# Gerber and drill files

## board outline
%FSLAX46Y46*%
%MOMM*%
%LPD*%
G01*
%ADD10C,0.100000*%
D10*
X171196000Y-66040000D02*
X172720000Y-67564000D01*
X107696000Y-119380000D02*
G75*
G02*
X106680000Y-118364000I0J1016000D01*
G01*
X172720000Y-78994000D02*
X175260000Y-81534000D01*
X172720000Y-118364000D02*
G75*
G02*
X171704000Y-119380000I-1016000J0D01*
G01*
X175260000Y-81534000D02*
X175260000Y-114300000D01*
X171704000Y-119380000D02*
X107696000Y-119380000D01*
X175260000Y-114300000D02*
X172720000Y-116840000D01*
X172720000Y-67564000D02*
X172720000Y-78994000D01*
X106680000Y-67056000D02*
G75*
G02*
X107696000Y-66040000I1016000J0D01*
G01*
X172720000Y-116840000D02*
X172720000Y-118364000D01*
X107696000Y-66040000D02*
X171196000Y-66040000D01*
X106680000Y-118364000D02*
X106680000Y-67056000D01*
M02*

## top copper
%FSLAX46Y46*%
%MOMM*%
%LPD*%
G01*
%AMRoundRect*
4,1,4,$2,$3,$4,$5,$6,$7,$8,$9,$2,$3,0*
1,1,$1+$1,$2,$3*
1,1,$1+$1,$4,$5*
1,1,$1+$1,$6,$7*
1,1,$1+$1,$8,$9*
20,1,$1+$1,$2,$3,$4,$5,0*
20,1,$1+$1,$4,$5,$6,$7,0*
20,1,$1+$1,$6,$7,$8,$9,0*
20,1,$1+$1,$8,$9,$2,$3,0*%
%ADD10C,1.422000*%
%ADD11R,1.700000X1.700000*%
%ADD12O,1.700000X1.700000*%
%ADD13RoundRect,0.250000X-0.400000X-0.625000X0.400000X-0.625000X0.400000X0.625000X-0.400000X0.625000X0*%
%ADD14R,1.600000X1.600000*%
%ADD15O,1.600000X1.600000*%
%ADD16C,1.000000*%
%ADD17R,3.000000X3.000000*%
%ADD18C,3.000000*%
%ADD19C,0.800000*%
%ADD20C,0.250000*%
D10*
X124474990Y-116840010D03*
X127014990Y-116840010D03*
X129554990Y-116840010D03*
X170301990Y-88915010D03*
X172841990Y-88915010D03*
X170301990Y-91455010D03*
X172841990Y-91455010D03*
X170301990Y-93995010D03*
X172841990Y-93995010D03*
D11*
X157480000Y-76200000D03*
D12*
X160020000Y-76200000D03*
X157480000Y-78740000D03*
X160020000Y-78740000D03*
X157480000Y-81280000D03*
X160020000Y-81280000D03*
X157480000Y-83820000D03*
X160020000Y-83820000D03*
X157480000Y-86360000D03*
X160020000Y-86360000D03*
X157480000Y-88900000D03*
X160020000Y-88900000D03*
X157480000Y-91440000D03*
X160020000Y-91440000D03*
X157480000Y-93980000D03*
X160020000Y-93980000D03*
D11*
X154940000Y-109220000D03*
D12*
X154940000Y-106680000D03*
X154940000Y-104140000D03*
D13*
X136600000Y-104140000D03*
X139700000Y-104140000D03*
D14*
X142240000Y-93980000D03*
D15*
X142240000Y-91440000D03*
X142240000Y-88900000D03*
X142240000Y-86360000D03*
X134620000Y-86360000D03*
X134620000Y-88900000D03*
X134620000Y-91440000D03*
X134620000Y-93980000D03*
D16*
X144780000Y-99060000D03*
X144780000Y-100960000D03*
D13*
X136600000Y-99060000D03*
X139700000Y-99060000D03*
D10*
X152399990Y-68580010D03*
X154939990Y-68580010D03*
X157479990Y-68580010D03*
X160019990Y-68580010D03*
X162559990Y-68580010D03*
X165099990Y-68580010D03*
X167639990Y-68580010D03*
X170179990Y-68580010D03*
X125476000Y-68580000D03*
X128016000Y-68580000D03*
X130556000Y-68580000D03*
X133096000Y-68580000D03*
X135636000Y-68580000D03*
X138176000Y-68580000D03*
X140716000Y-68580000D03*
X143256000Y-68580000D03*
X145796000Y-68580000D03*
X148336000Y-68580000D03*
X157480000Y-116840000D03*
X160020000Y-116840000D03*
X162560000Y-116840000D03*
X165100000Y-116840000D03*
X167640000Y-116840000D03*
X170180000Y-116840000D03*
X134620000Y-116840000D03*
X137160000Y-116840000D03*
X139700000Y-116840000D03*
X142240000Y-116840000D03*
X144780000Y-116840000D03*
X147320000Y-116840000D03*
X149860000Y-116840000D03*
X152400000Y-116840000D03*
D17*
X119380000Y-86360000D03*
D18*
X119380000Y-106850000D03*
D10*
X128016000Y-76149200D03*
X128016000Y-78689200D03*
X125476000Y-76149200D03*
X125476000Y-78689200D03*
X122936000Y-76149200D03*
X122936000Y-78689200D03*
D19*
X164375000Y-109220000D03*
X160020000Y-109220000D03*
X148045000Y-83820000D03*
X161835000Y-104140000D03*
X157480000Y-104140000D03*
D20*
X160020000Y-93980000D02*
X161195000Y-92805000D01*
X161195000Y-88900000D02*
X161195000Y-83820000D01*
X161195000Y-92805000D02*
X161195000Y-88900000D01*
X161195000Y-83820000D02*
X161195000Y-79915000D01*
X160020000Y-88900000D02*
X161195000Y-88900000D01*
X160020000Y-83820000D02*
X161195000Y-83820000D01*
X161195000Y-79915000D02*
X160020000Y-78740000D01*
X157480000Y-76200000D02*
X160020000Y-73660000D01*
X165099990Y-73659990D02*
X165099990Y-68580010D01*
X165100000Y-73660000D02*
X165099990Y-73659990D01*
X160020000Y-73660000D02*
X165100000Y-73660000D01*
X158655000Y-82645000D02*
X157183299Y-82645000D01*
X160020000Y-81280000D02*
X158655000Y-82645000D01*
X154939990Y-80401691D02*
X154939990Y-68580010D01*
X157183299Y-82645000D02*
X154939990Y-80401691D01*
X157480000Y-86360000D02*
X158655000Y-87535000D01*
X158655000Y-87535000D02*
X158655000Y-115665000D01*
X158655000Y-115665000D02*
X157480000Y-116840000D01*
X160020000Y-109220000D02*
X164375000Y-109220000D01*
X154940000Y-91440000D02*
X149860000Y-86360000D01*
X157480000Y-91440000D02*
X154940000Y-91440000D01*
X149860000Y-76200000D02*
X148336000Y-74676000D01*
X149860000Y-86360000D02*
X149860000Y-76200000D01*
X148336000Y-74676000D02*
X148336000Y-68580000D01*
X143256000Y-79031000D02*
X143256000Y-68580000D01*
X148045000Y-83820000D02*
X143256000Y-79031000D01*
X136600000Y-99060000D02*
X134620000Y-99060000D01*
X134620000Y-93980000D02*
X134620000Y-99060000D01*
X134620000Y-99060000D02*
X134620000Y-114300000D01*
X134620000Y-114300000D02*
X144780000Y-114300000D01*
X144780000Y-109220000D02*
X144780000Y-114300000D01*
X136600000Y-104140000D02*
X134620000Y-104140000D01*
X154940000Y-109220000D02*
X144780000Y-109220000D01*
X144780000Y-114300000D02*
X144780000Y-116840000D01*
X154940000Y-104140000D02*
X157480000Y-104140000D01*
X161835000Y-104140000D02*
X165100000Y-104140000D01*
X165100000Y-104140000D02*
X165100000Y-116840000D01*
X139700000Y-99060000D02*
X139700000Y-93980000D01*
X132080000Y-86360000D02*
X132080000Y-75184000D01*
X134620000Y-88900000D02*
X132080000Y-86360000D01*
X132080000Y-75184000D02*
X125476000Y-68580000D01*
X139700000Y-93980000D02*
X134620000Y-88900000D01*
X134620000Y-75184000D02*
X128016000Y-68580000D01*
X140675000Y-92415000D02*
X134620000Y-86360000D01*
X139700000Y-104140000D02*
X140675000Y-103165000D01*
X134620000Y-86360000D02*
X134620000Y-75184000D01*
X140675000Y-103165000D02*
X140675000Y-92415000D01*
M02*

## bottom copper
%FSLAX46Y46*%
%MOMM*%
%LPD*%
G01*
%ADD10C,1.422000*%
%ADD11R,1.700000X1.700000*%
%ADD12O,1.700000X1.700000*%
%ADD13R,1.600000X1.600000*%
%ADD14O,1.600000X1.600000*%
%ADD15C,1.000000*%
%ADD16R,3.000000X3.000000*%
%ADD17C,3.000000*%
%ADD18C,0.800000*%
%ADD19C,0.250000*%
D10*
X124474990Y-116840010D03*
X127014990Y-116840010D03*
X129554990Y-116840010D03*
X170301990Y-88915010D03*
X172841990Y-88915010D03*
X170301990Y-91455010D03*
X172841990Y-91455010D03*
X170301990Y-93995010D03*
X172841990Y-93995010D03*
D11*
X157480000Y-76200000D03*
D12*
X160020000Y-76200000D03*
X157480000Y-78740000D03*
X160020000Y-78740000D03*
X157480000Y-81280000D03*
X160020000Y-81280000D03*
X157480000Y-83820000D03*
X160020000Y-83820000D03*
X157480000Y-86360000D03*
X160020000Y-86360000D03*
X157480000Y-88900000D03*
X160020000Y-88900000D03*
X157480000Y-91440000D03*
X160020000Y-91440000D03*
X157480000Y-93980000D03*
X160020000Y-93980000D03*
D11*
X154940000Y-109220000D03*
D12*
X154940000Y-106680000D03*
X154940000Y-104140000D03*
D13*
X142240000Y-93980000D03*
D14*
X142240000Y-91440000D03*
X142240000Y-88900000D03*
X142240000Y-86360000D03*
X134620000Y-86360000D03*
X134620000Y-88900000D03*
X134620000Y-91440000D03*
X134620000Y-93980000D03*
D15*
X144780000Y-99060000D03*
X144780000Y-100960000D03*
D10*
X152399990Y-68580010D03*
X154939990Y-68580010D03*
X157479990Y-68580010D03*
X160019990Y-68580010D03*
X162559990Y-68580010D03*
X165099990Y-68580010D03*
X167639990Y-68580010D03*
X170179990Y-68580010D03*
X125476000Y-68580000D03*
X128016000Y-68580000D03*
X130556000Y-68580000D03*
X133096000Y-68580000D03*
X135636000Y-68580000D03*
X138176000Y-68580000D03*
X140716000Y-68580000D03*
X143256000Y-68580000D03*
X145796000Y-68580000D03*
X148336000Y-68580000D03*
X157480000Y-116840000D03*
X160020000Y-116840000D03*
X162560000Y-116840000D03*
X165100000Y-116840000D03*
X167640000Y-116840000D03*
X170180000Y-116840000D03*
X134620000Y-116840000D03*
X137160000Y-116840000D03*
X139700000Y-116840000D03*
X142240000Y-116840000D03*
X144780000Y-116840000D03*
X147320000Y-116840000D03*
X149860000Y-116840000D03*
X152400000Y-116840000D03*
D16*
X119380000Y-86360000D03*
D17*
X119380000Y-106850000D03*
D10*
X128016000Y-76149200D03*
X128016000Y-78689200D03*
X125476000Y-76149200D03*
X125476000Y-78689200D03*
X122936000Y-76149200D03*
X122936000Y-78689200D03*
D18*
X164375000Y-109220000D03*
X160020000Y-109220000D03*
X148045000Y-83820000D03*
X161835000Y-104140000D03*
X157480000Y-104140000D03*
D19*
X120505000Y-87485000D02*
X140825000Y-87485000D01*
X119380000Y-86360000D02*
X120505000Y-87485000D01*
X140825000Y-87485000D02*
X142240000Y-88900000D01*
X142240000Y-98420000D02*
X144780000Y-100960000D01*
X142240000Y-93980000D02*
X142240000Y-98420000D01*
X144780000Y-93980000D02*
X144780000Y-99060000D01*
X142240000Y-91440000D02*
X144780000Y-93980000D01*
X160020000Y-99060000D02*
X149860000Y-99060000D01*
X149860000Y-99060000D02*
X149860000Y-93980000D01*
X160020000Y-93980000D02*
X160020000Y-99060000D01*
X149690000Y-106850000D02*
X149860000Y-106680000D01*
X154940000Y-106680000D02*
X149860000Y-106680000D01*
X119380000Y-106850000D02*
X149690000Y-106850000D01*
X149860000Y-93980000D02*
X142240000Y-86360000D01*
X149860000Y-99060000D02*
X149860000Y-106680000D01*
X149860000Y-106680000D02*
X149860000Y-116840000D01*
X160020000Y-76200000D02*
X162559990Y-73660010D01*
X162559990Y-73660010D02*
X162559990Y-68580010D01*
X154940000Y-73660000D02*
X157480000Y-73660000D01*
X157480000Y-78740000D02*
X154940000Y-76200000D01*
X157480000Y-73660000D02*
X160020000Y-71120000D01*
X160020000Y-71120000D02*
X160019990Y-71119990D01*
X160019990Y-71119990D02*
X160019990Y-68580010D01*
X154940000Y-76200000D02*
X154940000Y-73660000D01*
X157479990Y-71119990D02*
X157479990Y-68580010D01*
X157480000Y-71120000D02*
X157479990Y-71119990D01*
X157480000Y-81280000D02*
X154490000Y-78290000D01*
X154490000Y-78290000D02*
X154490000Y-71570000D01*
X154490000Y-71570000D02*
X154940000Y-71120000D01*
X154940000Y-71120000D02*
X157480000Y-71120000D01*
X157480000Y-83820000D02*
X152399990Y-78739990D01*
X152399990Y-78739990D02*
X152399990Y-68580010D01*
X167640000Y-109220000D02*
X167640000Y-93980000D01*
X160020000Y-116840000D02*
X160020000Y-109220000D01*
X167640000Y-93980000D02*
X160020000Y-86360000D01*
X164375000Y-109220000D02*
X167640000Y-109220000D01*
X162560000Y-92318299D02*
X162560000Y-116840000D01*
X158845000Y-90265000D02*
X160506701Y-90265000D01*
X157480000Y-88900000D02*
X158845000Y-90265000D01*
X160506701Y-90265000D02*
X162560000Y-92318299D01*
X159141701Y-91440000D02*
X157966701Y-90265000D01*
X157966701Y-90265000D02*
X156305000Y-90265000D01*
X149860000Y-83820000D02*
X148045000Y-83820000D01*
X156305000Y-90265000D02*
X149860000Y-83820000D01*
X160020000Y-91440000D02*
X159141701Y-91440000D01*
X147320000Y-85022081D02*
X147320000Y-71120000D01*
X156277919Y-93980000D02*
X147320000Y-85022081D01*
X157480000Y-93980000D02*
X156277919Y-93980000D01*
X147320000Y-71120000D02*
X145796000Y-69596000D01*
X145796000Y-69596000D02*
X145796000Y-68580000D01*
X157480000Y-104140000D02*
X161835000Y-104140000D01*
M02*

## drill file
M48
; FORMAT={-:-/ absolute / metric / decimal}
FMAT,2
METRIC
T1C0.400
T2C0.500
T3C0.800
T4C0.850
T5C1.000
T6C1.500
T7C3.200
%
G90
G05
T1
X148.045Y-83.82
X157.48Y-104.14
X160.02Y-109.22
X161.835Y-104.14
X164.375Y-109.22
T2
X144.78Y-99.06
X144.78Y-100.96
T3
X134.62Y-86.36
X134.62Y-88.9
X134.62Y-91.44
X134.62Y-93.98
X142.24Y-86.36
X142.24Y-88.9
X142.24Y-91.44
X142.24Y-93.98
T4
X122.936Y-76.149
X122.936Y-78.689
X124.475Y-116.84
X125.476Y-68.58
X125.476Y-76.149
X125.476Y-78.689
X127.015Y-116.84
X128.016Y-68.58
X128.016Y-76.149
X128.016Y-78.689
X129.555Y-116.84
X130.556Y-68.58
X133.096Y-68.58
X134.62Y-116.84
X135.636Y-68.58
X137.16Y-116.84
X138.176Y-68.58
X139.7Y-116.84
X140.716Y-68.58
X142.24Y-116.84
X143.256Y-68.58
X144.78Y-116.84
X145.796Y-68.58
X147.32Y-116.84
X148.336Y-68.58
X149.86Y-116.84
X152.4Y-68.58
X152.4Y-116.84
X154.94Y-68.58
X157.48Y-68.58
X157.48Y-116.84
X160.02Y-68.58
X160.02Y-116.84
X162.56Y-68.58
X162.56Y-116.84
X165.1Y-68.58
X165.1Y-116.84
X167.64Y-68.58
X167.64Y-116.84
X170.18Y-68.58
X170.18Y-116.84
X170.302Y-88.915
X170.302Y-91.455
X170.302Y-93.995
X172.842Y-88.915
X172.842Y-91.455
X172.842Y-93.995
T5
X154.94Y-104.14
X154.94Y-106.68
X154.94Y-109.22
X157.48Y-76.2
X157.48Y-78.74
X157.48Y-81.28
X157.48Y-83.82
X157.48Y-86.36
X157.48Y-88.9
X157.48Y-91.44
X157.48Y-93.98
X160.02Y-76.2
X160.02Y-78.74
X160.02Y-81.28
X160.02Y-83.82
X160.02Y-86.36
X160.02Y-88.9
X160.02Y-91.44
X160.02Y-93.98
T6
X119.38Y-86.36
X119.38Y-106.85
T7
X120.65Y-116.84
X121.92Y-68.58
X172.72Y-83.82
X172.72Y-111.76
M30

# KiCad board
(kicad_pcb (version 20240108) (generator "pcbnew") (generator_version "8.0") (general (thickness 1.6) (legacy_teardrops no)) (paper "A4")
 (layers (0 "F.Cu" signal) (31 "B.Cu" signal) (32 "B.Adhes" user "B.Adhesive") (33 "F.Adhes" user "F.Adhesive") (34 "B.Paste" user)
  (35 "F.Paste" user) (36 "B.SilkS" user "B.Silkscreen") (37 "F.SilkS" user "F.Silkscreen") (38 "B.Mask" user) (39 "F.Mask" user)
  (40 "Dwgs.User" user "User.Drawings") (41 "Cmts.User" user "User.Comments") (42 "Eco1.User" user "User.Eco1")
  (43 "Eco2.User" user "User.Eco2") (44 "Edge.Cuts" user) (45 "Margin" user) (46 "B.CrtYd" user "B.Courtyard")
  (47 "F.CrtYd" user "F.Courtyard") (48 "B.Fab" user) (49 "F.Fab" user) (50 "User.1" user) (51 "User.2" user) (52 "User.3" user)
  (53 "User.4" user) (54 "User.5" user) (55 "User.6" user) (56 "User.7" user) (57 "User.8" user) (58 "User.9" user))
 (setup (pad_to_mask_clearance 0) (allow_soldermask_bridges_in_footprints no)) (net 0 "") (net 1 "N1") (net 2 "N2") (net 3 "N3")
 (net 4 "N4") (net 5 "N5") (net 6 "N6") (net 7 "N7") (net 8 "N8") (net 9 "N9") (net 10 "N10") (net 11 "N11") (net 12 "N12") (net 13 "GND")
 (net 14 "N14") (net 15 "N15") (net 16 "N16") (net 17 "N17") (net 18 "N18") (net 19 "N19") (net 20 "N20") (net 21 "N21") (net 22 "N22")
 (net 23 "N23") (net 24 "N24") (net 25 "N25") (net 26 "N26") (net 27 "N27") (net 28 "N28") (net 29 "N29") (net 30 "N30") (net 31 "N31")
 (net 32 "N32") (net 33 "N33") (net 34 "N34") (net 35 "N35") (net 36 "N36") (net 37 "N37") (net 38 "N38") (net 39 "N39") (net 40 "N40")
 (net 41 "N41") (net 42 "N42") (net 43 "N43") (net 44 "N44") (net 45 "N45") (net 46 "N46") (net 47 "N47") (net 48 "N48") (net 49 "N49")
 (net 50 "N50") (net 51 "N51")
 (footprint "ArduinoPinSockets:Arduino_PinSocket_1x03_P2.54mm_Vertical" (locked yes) (layer "F.Cu") (at 124.47499 116.84001 90)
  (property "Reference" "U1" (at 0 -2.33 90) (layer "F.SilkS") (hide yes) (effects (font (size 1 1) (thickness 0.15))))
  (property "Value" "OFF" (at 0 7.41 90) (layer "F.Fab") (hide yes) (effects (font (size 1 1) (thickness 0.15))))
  (pad "1" thru_hole circle (at 0 0 90) (size 1.422 1.422) (drill 0.85) (layers "*.Cu" "*.Mask") (remove_unused_layers no) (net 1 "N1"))
  (pad "2" thru_hole circle (at 0 2.54 90) (size 1.422 1.422) (drill 0.85) (layers "*.Cu" "*.Mask") (remove_unused_layers no) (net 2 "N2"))
  (pad "3" thru_hole circle (at 0 5.08 90) (size 1.422 1.422) (drill 0.85) (layers "*.Cu" "*.Mask") (remove_unused_layers no) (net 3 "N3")))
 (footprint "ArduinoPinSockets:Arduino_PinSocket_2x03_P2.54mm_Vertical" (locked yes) (layer "F.Cu") (at 170.30199 88.91501)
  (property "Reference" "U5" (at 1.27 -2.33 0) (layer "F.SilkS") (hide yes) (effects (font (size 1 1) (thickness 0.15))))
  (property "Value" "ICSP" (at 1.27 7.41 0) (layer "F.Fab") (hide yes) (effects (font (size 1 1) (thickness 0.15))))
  (pad "1" thru_hole circle (at 0 0) (size 1.422 1.422) (drill 0.85) (layers "*.Cu" "*.Mask") (remove_unused_layers no) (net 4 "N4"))
  (pad "2" thru_hole circle (at 2.54 0) (size 1.422 1.422) (drill 0.85) (layers "*.Cu" "*.Mask") (remove_unused_layers no) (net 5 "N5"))
  (pad "3" thru_hole circle (at 0 2.54) (size 1.422 1.422) (drill 0.85) (layers "*.Cu" "*.Mask") (remove_unused_layers no) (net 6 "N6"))
  (pad "4" thru_hole circle (at 2.54 2.54) (size 1.422 1.422) (drill 0.85) (layers "*.Cu" "*.Mask") (remove_unused_layers no) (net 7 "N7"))
  (pad "5" thru_hole circle (at 0 5.08) (size 1.422 1.422) (drill 0.85) (layers "*.Cu" "*.Mask") (remove_unused_layers no) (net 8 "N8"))
  (pad "6" thru_hole circle (at 2.54 5.08) (size 1.422 1.422) (drill 0.85) (layers "*.Cu" "*.Mask") (remove_unused_layers no) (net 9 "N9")))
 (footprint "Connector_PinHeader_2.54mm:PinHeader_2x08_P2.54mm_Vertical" (layer "F.Cu") (at 157.48 76.2)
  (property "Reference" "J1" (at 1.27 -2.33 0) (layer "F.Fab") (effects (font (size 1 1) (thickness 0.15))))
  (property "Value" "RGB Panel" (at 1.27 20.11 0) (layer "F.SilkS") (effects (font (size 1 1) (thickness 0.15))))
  (pad "1" thru_hole rect (at 0 0) (size 1.7 1.7) (drill 1) (layers "*.Cu" "*.Mask") (remove_unused_layers no) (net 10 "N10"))
  (pad "2" thru_hole oval (at 2.54 0) (size 1.7 1.7) (drill 1) (layers "*.Cu" "*.Mask") (remove_unused_layers no) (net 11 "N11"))
  (pad "3" thru_hole oval (at 0 2.54) (size 1.7 1.7) (drill 1) (layers "*.Cu" "*.Mask") (remove_unused_layers no) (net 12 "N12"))
  (pad "4" thru_hole oval (at 2.54 2.54) (size 1.7 1.7) (drill 1) (layers "*.Cu" "*.Mask") (remove_unused_layers no) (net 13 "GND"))
  (pad "5" thru_hole oval (at 0 5.08) (size 1.7 1.7) (drill 1) (layers "*.Cu" "*.Mask") (remove_unused_layers no) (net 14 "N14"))
  (pad "6" thru_hole oval (at 2.54 5.08) (size 1.7 1.7) (drill 1) (layers "*.Cu" "*.Mask") (remove_unused_layers no) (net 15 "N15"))
  (pad "7" thru_hole oval (at 0 7.62) (size 1.7 1.7) (drill 1) (layers "*.Cu" "*.Mask") (remove_unused_layers no) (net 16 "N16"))
  (pad "8" thru_hole oval (at 2.54 7.62) (size 1.7 1.7) (drill 1) (layers "*.Cu" "*.Mask") (remove_unused_layers no) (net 13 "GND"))
  (pad "9" thru_hole oval (at 0 10.16) (size 1.7 1.7) (drill 1) (layers "*.Cu" "*.Mask") (remove_unused_layers no) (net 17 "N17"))
  (pad "10" thru_hole oval (at 2.54 10.16) (size 1.7 1.7) (drill 1) (layers "*.Cu" "*.Mask") (remove_unused_layers no) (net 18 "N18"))
  (pad "11" thru_hole oval (at 0 12.7) (size 1.7 1.7) (drill 1) (layers "*.Cu" "*.Mask") (remove_unused_layers no) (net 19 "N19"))
  (pad "12" thru_hole oval (at 2.54 12.7) (size 1.7 1.7) (drill 1) (layers "*.Cu" "*.Mask") (remove_unused_layers no) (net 15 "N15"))
  (pad "13" thru_hole oval (at 0 15.24) (size 1.7 1.7) (drill 1) (layers "*.Cu" "*.Mask") (remove_unused_layers no) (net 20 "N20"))
  (pad "14" thru_hole oval (at 2.54 15.24) (size 1.7 1.7) (drill 1) (layers "*.Cu" "*.Mask") (remove_unused_layers no) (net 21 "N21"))
  (pad "15" thru_hole oval (at 0 17.78) (size 1.7 1.7) (drill 1) (layers "*.Cu" "*.Mask") (remove_unused_layers no) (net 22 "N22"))
  (pad "16" thru_hole oval (at 2.54 17.78) (size 1.7 1.7) (drill 1) (layers "*.Cu" "*.Mask") (remove_unused_layers no) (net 13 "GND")))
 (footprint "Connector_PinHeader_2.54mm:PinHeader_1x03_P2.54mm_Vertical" (layer "F.Cu") (at 154.94 109.22 180)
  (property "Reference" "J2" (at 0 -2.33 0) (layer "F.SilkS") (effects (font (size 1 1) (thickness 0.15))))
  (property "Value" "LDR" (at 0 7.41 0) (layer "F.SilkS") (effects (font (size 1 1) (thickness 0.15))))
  (pad "1" thru_hole rect (at 0 0 180) (size 1.7 1.7) (drill 1) (layers "*.Cu" "*.Mask") (remove_unused_layers no) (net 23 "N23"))
  (pad "2" thru_hole oval (at 0 2.54 180) (size 1.7 1.7) (drill 1) (layers "*.Cu" "*.Mask") (remove_unused_layers no) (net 13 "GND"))
  (pad "3" thru_hole oval (at 0 5.08 180) (size 1.7 1.7) (drill 1) (layers "*.Cu" "*.Mask") (remove_unused_layers no) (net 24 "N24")))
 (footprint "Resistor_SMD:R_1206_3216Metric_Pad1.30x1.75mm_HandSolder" (layer "F.Cu") (at 138.15 104.14)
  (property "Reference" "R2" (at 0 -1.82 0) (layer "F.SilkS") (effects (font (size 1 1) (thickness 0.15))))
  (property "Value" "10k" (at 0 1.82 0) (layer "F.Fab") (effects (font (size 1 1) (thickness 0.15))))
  (pad "1" smd roundrect (at -1.55 0) (size 1.3 1.75) (layers "F.Cu" "F.Paste" "F.Mask") (roundrect_rratio 0.1923076923) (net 23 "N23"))
  (pad "2" smd roundrect (at 1.55 0) (size 1.3 1.75) (layers "F.Cu" "F.Paste" "F.Mask") (roundrect_rratio 0.1923076923) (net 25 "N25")))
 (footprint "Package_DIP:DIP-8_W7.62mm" (layer "F.Cu") (at 142.24 93.98 180)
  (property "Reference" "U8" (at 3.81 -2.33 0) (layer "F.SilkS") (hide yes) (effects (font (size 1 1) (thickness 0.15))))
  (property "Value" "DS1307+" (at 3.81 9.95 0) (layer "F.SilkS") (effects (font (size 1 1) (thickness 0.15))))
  (pad "1" thru_hole rect (at 0 0 180) (size 1.6 1.6) (drill 0.8) (layers "*.Cu" "*.Mask") (remove_unused_layers no) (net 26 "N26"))
  (pad "2" thru_hole oval (at 0 2.54 180) (size 1.6 1.6) (drill 0.8) (layers "*.Cu" "*.Mask") (remove_unused_layers no) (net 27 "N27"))
  (pad "3" thru_hole oval (at 0 5.08 180) (size 1.6 1.6) (drill 0.8) (layers "*.Cu" "*.Mask") (remove_unused_layers no) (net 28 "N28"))
  (pad "4" thru_hole oval (at 0 7.62 180) (size 1.6 1.6) (drill 0.8) (layers "*.Cu" "*.Mask") (remove_unused_layers no) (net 13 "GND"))
  (pad "5" thru_hole oval (at 7.62 7.62 180) (size 1.6 1.6) (drill 0.8) (layers "*.Cu" "*.Mask") (remove_unused_layers no) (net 25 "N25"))
  (pad "6" thru_hole oval (at 7.62 5.08 180) (size 1.6 1.6) (drill 0.8) (layers "*.Cu" "*.Mask") (remove_unused_layers no) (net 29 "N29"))
  (pad "7" thru_hole oval (at 7.62 2.54 180) (size 1.6 1.6) (drill 0.8) (layers "*.Cu" "*.Mask") (remove_unused_layers no) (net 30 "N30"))
  (pad "8" thru_hole oval (at 7.62 0 180) (size 1.6 1.6) (drill 0.8) (layers "*.Cu" "*.Mask") (remove_unused_layers no) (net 23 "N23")))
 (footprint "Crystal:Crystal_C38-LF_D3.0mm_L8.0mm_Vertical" (layer "F.Cu") (at 144.78 99.06 -90)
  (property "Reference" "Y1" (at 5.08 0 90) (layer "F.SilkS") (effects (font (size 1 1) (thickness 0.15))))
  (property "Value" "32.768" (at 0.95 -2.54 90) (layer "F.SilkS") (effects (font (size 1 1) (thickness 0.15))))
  (pad "1" thru_hole circle (at 0 0 270) (size 1 1) (drill 0.5) (layers "*.Cu" "*.Mask") (remove_unused_layers no) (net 27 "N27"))
  (pad "2" thru_hole circle (at 1.9 0 270) (size 1 1) (drill 0.5) (layers "*.Cu" "*.Mask") (remove_unused_layers no) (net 26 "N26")))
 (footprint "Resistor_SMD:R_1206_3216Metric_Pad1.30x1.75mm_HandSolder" (layer "F.Cu") (at 138.15 99.06)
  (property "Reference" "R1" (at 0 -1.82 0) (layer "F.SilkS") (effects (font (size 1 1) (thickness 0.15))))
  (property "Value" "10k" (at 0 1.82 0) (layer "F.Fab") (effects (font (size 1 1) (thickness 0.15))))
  (pad "1" smd roundrect (at -1.55 0) (size 1.3 1.75) (layers "F.Cu" "F.Paste" "F.Mask") (roundrect_rratio 0.1923076923) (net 23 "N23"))
  (pad "2" smd roundrect (at 1.55 0) (size 1.3 1.75) (layers "F.Cu" "F.Paste" "F.Mask") (roundrect_rratio 0.1923076923) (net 29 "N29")))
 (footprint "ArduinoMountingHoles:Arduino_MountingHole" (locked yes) (layer "F.Cu") (at 172.72 83.82001)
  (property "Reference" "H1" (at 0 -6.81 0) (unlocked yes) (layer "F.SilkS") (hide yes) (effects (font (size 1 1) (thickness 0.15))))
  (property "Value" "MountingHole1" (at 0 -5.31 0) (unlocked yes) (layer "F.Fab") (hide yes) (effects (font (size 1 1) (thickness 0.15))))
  (pad "" np_thru_hole circle (at 0 0) (size 3.19989 3.19989) (drill 3.19989) (layers "F&B.Cu" "*.Mask") (solder_mask_margin 0.5)))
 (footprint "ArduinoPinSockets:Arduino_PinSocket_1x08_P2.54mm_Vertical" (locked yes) (layer "F.Cu") (at 152.39999 68.58001 90)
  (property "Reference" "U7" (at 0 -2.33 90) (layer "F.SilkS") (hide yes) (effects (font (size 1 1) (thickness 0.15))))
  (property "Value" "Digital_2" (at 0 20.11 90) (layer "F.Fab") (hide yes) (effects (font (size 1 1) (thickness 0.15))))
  (pad "11" thru_hole circle (at 0 0 90) (size 1.422 1.422) (drill 0.85) (layers "*.Cu" "*.Mask") (remove_unused_layers no) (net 16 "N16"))
  (pad "12" thru_hole circle (at 0 2.54 90) (size 1.422 1.422) (drill 0.85) (layers "*.Cu" "*.Mask") (remove_unused_layers no)
   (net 15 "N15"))
  (pad "13" thru_hole circle (at 0 5.08 90) (size 1.422 1.422) (drill 0.85) (layers "*.Cu" "*.Mask") (remove_unused_layers no)
   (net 14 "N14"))
  (pad "14" thru_hole circle (at 0 7.62 90) (size 1.422 1.422) (drill 0.85) (layers "*.Cu" "*.Mask") (remove_unused_layers no)
   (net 12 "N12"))
  (pad "15" thru_hole circle (at 0 10.16 90) (size 1.422 1.422) (drill 0.85) (layers "*.Cu" "*.Mask") (remove_unused_layers no)
   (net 11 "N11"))
  (pad "16" thru_hole circle (at 0 12.7 90) (size 1.422 1.422) (drill 0.85) (layers "*.Cu" "*.Mask") (remove_unused_layers no)
   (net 10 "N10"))
  (pad "17" thru_hole circle (at 0 15.24 90) (size 1.422 1.422) (drill 0.85) (layers "*.Cu" "*.Mask") (remove_unused_layers no)
   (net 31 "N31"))
  (pad "18" thru_hole circle (at 0 17.78 90) (size 1.422 1.422) (drill 0.85) (layers "*.Cu" "*.Mask") (remove_unused_layers no)
   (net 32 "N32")))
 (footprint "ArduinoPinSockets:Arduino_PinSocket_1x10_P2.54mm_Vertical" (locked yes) (layer "F.Cu") (at 125.476 68.58 90)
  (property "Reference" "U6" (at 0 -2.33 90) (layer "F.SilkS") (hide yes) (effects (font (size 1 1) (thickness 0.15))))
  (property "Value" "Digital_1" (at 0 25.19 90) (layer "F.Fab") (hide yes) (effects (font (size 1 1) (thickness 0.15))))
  (pad "1" thru_hole circle (at 0 0 90) (size 1.422 1.422) (drill 0.85) (layers "*.Cu" "*.Mask") (remove_unused_layers no) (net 29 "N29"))
  (pad "2" thru_hole circle (at 0 2.54 90) (size 1.422 1.422) (drill 0.85) (layers "*.Cu" "*.Mask") (remove_unused_layers no) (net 25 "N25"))
  (pad "3" thru_hole circle (at 0 5.08 90) (size 1.422 1.422) (drill 0.85) (layers "*.Cu" "*.Mask") (remove_unused_layers no) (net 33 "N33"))
  (pad "4" thru_hole circle (at 0 7.62 90) (size 1.422 1.422) (drill 0.85) (layers "*.Cu" "*.Mask") (remove_unused_layers no) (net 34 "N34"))
  (pad "5" thru_hole circle (at 0 10.16 90) (size 1.422 1.422) (drill 0.85) (layers "*.Cu" "*.Mask") (remove_unused_layers no)
   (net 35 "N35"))
  (pad "6" thru_hole circle (at 0 12.7 90) (size 1.422 1.422) (drill 0.85) (layers "*.Cu" "*.Mask") (remove_unused_layers no) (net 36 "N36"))
  (pad "7" thru_hole circle (at 0 15.24 90) (size 1.422 1.422) (drill 0.85) (layers "*.Cu" "*.Mask") (remove_unused_layers no)
   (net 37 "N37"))
  (pad "8" thru_hole circle (at 0 17.78 90) (size 1.422 1.422) (drill 0.85) (layers "*.Cu" "*.Mask") (remove_unused_layers no)
   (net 21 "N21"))
  (pad "9" thru_hole circle (at 0 20.32 90) (size 1.422 1.422) (drill 0.85) (layers "*.Cu" "*.Mask") (remove_unused_layers no)
   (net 22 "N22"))
  (pad "10" thru_hole circle (at 0 22.86 90) (size 1.422 1.422) (drill 0.85) (layers "*.Cu" "*.Mask") (remove_unused_layers no)
   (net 20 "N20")))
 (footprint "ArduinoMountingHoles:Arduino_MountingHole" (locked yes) (layer "F.Cu") (at 120.65 116.84)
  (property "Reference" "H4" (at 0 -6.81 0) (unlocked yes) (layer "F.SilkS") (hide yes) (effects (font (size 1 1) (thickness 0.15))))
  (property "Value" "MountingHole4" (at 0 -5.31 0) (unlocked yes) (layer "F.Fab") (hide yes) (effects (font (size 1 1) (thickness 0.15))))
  (pad "" np_thru_hole circle (at 0 0) (size 3.19989 3.19989) (drill 3.19989) (layers "F&B.Cu" "*.Mask") (solder_mask_margin 0.5)))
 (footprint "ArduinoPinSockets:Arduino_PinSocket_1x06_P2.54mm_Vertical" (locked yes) (layer "F.Cu") (at 157.48 116.84 90)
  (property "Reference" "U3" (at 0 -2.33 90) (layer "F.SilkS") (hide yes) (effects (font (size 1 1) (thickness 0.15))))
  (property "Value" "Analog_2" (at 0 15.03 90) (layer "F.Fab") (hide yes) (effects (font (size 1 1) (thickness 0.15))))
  (pad "9" thru_hole circle (at 0 0 90) (size 1.422 1.422) (drill 0.85) (layers "*.Cu" "*.Mask") (remove_unused_layers no) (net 17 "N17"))
  (pad "10" thru_hole circle (at 0 2.54 90) (size 1.422 1.422) (drill 0.85) (layers "*.Cu" "*.Mask") (remove_unused_layers no)
   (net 18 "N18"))
  (pad "11" thru_hole circle (at 0 5.08 90) (size 1.422 1.422) (drill 0.85) (layers "*.Cu" "*.Mask") (remove_unused_layers no)
   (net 19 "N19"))
  (pad "12" thru_hole circle (at 0 7.62 90) (size 1.422 1.422) (drill 0.85) (layers "*.Cu" "*.Mask") (remove_unused_layers no)
   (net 24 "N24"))
  (pad "13" thru_hole circle (at 0 10.16 90) (size 1.422 1.422) (drill 0.85) (layers "*.Cu" "*.Mask") (remove_unused_layers no)
   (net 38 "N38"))
  (pad "14" thru_hole circle (at 0 12.7 90) (size 1.422 1.422) (drill 0.85) (layers "*.Cu" "*.Mask") (remove_unused_layers no)
   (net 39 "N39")))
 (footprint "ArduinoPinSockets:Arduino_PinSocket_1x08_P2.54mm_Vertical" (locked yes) (layer "F.Cu") (at 134.62 116.84 90)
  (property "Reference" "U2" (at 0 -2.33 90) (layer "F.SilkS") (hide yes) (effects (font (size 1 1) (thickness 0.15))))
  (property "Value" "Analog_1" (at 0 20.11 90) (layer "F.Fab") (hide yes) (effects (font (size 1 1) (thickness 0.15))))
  (pad "1" thru_hole circle (at 0 0 90) (size 1.422 1.422) (drill 0.85) (layers "*.Cu" "*.Mask") (remove_unused_layers no) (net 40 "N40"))
  (pad "2" thru_hole circle (at 0 2.54 90) (size 1.422 1.422) (drill 0.85) (layers "*.Cu" "*.Mask") (remove_unused_layers no) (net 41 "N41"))
  (pad "3" thru_hole circle (at 0 5.08 90) (size 1.422 1.422) (drill 0.85) (layers "*.Cu" "*.Mask") (remove_unused_layers no) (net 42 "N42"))
  (pad "4" thru_hole circle (at 0 7.62 90) (size 1.422 1.422) (drill 0.85) (layers "*.Cu" "*.Mask") (remove_unused_layers no) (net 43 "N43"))
  (pad "5" thru_hole circle (at 0 10.16 90) (size 1.422 1.422) (drill 0.85) (layers "*.Cu" "*.Mask") (remove_unused_layers no)
   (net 23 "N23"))
  (pad "6" thru_hole circle (at 0 12.7 90) (size 1.422 1.422) (drill 0.85) (layers "*.Cu" "*.Mask") (remove_unused_layers no) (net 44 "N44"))
  (pad "7" thru_hole circle (at 0 15.24 90) (size 1.422 1.422) (drill 0.85) (layers "*.Cu" "*.Mask") (remove_unused_layers no)
   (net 13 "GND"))
  (pad "8" thru_hole circle (at 0 17.78 90) (size 1.422 1.422) (drill 0.85) (layers "*.Cu" "*.Mask") (remove_unused_layers no)
   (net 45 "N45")))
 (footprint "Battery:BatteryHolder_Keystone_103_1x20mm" (layer "F.Cu") (at 119.38 86.36 -90)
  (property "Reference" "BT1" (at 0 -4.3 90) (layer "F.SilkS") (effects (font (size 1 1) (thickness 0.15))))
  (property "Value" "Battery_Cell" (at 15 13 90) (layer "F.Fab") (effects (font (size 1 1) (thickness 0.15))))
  (pad "1" thru_hole rect (at 0 0 270) (size 3 3) (drill 1.5) (layers "*.Cu" "*.Mask") (remove_unused_layers no) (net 28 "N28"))
  (pad "2" thru_hole circle (at 20.49 0 270) (size 3 3) (drill 1.5) (layers "*.Cu" "*.Mask") (remove_unused_layers no) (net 13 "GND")))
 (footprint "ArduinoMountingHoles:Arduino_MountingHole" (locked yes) (layer "F.Cu") (at 121.91999 68.58001)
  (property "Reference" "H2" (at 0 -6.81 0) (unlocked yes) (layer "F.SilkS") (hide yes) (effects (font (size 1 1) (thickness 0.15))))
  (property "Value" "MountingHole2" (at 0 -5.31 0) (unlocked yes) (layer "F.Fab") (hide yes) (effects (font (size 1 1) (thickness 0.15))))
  (pad "" np_thru_hole circle (at 0 0) (size 3.19989 3.19989) (drill 3.19989) (layers "F&B.Cu" "*.Mask") (solder_mask_margin 0.5)))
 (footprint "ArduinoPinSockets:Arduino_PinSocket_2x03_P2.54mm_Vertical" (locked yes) (layer "F.Cu") (at 128.016 76.1492 -90)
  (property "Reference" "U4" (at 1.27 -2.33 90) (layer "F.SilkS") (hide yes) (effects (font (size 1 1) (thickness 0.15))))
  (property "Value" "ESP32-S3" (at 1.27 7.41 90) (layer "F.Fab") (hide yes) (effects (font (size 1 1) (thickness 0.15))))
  (pad "1" thru_hole circle (at 0 0 270) (size 1.422 1.422) (drill 0.85) (layers "*.Cu" "*.Mask") (remove_unused_layers no) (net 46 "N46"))
  (pad "2" thru_hole circle (at 2.54 0 270) (size 1.422 1.422) (drill 0.85) (layers "*.Cu" "*.Mask") (remove_unused_layers no)
   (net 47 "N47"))
  (pad "3" thru_hole circle (at 0 2.54 270) (size 1.422 1.422) (drill 0.85) (layers "*.Cu" "*.Mask") (remove_unused_layers no)
   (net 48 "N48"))
  (pad "4" thru_hole circle (at 2.54 2.54 270) (size 1.422 1.422) (drill 0.85) (layers "*.Cu" "*.Mask") (remove_unused_layers no)
   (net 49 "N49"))
  (pad "5" thru_hole circle (at 0 5.08 270) (size 1.422 1.422) (drill 0.85) (layers "*.Cu" "*.Mask") (remove_unused_layers no)
   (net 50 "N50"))
  (pad "6" thru_hole circle (at 2.54 5.08 270) (size 1.422 1.422) (drill 0.85) (layers "*.Cu" "*.Mask") (remove_unused_layers no)
   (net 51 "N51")))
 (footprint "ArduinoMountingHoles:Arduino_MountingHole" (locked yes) (layer "F.Cu") (at 172.72 111.76)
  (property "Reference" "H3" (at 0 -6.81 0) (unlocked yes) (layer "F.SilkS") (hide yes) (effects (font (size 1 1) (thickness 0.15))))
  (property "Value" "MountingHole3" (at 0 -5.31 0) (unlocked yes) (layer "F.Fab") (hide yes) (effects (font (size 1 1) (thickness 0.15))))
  (pad "" np_thru_hole circle (at 0 0) (size 3.19989 3.19989) (drill 3.19989) (layers "F&B.Cu" "*.Mask") (solder_mask_margin 0.5)))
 (gr_line (start 171.196 66.04) (end 172.72 67.564) (locked yes) (stroke (width 0.1) (type solid)) (layer "Edge.Cuts"))
 (gr_arc (start 107.696 119.38) (mid 106.97758 119.08242) (end 106.68 118.364) (locked yes) (stroke (width 0.1) (type solid))
  (layer "Edge.Cuts"))
 (gr_line (start 172.72 78.994) (end 175.26 81.534) (locked yes) (stroke (width 0.1) (type solid)) (layer "Edge.Cuts"))
 (gr_arc (start 172.72 118.364) (mid 172.42242 119.08242) (end 171.704 119.38) (locked yes) (stroke (width 0.1) (type solid))
  (layer "Edge.Cuts"))
 (gr_line (start 175.26 81.534) (end 175.26 114.3) (locked yes) (stroke (width 0.1) (type solid)) (layer "Edge.Cuts"))
 (gr_line (start 171.704 119.38) (end 107.696 119.38) (locked yes) (stroke (width 0.1) (type solid)) (layer "Edge.Cuts"))
 (gr_line (start 175.26 114.3) (end 172.72 116.84) (locked yes) (stroke (width 0.1) (type solid)) (layer "Edge.Cuts"))
 (gr_line (start 172.72 67.564) (end 172.72 78.994) (locked yes) (stroke (width 0.1) (type solid)) (layer "Edge.Cuts"))
 (gr_arc (start 106.68 67.056) (mid 106.97758 66.33758) (end 107.696 66.04) (locked yes) (stroke (width 0.1) (type solid))
  (layer "Edge.Cuts"))
 (gr_line (start 172.72 116.84) (end 172.72 118.364) (locked yes) (stroke (width 0.1) (type solid)) (layer "Edge.Cuts"))
 (gr_line (start 107.696 66.04) (end 171.196 66.04) (locked yes) (stroke (width 0.1) (type solid)) (layer "Edge.Cuts"))
 (gr_line (start 106.68 118.364) (end 106.68 67.056) (locked yes) (stroke (width 0.1) (type solid)) (layer "Edge.Cuts"))
 (segment (start 120.505 87.485) (end 140.825 87.485) (width 0.25) (layer "B.Cu") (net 28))
 (segment (start 119.38 86.36) (end 120.505 87.485) (width 0.25) (layer "B.Cu") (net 28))
 (segment (start 140.825 87.485) (end 142.24 88.9) (width 0.25) (layer "B.Cu") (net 28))
 (segment (start 142.24 98.42) (end 144.78 100.96) (width 0.25) (layer "B.Cu") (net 26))
 (segment (start 142.24 93.98) (end 142.24 98.42) (width 0.25) (layer "B.Cu") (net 26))
 (segment (start 144.78 93.98) (end 144.78 99.06) (width 0.25) (layer "B.Cu") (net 27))
 (segment (start 142.24 91.44) (end 144.78 93.98) (width 0.25) (layer "B.Cu") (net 27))
 (segment (start 160.02 93.98) (end 161.195 92.805) (width 0.25) (layer "F.Cu") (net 13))
 (segment (start 161.195 88.9) (end 161.195 83.82) (width 0.25) (layer "F.Cu") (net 13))
 (segment (start 161.195 92.805) (end 161.195 88.9) (width 0.25) (layer "F.Cu") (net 13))
 (segment (start 161.195 83.82) (end 161.195 79.915) (width 0.25) (layer "F.Cu") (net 13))
 (segment (start 160.02 88.9) (end 161.195 88.9) (width 0.25) (layer "F.Cu") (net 13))
 (segment (start 160.02 83.82) (end 161.195 83.82) (width 0.25) (layer "F.Cu") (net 13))
 (segment (start 161.195 79.915) (end 160.02 78.74) (width 0.25) (layer "F.Cu") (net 13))
 (segment (start 160.02 99.06) (end 149.86 99.06) (width 0.25) (layer "B.Cu") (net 13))
 (segment (start 149.86 99.06) (end 149.86 93.98) (width 0.25) (layer "B.Cu") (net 13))
 (segment (start 160.02 93.98) (end 160.02 99.06) (width 0.25) (layer "B.Cu") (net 13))
 (segment (start 149.69 106.85) (end 149.86 106.68) (width 0.25) (layer "B.Cu") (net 13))
 (segment (start 154.94 106.68) (end 149.86 106.68) (width 0.25) (layer "B.Cu") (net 13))
 (segment (start 119.38 106.85) (end 149.69 106.85) (width 0.25) (layer "B.Cu") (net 13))
 (segment (start 149.86 93.98) (end 142.24 86.36) (width 0.25) (layer "B.Cu") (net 13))
 (segment (start 149.86 99.06) (end 149.86 106.68) (width 0.25) (layer "B.Cu") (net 13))
 (segment (start 149.86 106.68) (end 149.86 116.84) (width 0.25) (layer "B.Cu") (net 13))
 (segment (start 157.48 76.2) (end 160.02 73.66) (width 0.25) (layer "F.Cu") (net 10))
 (segment (start 165.09999 73.65999) (end 165.09999 68.58001) (width 0.25) (layer "F.Cu") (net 10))
 (segment (start 165.1 73.66) (end 165.09999 73.65999) (width 0.25) (layer "F.Cu") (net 10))
 (segment (start 160.02 73.66) (end 165.1 73.66) (width 0.25) (layer "F.Cu") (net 10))
 (segment (start 160.02 76.2) (end 162.55999 73.66001) (width 0.25) (layer "B.Cu") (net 11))
 (segment (start 162.55999 73.66001) (end 162.55999 68.58001) (width 0.25) (layer "B.Cu") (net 11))
 (segment (start 154.94 73.66) (end 157.48 73.66) (width 0.25) (layer "B.Cu") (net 12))
 (segment (start 157.48 78.74) (end 154.94 76.2) (width 0.25) (layer "B.Cu") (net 12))
 (segment (start 157.48 73.66) (end 160.02 71.12) (width 0.25) (layer "B.Cu") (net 12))
 (segment (start 160.02 71.12) (end 160.01999 71.11999) (width 0.25) (layer "B.Cu") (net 12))
 (segment (start 160.01999 71.11999) (end 160.01999 68.58001) (width 0.25) (layer "B.Cu") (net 12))
 (segment (start 154.94 76.2) (end 154.94 73.66) (width 0.25) (layer "B.Cu") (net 12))
 (segment (start 157.47999 71.11999) (end 157.47999 68.58001) (width 0.25) (layer "B.Cu") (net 14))
 (segment (start 157.48 71.12) (end 157.47999 71.11999) (width 0.25) (layer "B.Cu") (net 14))
 (segment (start 157.48 81.28) (end 154.49 78.29) (width 0.25) (layer "B.Cu") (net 14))
 (segment (start 154.49 78.29) (end 154.49 71.57) (width 0.25) (layer "B.Cu") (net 14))
 (segment (start 154.49 71.57) (end 154.94 71.12) (width 0.25) (layer "B.Cu") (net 14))
 (segment (start 154.94 71.12) (end 157.48 71.12) (width 0.25) (layer "B.Cu") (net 14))
 (segment (start 158.655 82.645) (end 157.183299 82.645) (width 0.25) (layer "F.Cu") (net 15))
 (segment (start 160.02 81.28) (end 158.655 82.645) (width 0.25) (layer "F.Cu") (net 15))
 (segment (start 154.93999 80.401691) (end 154.93999 68.58001) (width 0.25) (layer "F.Cu") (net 15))
 (segment (start 157.183299 82.645) (end 154.93999 80.401691) (width 0.25) (layer "F.Cu") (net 15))
 (segment (start 157.48 83.82) (end 152.39999 78.73999) (width 0.25) (layer "B.Cu") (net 16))
 (segment (start 152.39999 78.73999) (end 152.39999 68.58001) (width 0.25) (layer "B.Cu") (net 16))
 (segment (start 157.48 86.36) (end 158.655 87.535) (width 0.25) (layer "F.Cu") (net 17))
 (segment (start 158.655 87.535) (end 158.655 115.665) (width 0.25) (layer "F.Cu") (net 17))
 (segment (start 158.655 115.665) (end 157.48 116.84) (width 0.25) (layer "F.Cu") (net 17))
 (segment (start 160.02 109.22) (end 164.375 109.22) (width 0.25) (layer "F.Cu") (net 18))
 (via (at 164.375 109.22) (size 0.8) (drill 0.4) (layers "F.Cu" "B.Cu") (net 18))
 (via (at 160.02 109.22) (size 0.8) (drill 0.4) (layers "F.Cu" "B.Cu") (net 18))
 (segment (start 167.64 109.22) (end 167.64 93.98) (width 0.25) (layer "B.Cu") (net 18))
 (segment (start 160.02 116.84) (end 160.02 109.22) (width 0.25) (layer "B.Cu") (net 18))
 (segment (start 167.64 93.98) (end 160.02 86.36) (width 0.25) (layer "B.Cu") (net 18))
 (segment (start 164.375 109.22) (end 167.64 109.22) (width 0.25) (layer "B.Cu") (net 18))
 (segment (start 162.56 92.318299) (end 162.56 116.84) (width 0.25) (layer "B.Cu") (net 19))
 (segment (start 158.845 90.265) (end 160.506701 90.265) (width 0.25) (layer "B.Cu") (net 19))
 (segment (start 157.48 88.9) (end 158.845 90.265) (width 0.25) (layer "B.Cu") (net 19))
 (segment (start 160.506701 90.265) (end 162.56 92.318299) (width 0.25) (layer "B.Cu") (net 19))
 (segment (start 154.94 91.44) (end 149.86 86.36) (width 0.25) (layer "F.Cu") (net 20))
 (segment (start 157.48 91.44) (end 154.94 91.44) (width 0.25) (layer "F.Cu") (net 20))
 (segment (start 149.86 76.2) (end 148.336 74.676) (width 0.25) (layer "F.Cu") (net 20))
 (segment (start 149.86 86.36) (end 149.86 76.2) (width 0.25) (layer "F.Cu") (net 20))
 (segment (start 148.336 74.676) (end 148.336 68.58) (width 0.25) (layer "F.Cu") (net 20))
 (segment (start 143.256 79.031) (end 143.256 68.58) (width 0.25) (layer "F.Cu") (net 21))
 (segment (start 148.045 83.82) (end 143.256 79.031) (width 0.25) (layer "F.Cu") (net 21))
 (via (at 148.045 83.82) (size 0.8) (drill 0.4) (layers "F.Cu" "B.Cu") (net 21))
 (segment (start 159.141701 91.44) (end 157.966701 90.265) (width 0.25) (layer "B.Cu") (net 21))
 (segment (start 157.966701 90.265) (end 156.305 90.265) (width 0.25) (layer "B.Cu") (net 21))
 (segment (start 149.86 83.82) (end 148.045 83.82) (width 0.25) (layer "B.Cu") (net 21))
 (segment (start 156.305 90.265) (end 149.86 83.82) (width 0.25) (layer "B.Cu") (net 21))
 (segment (start 160.02 91.44) (end 159.141701 91.44) (width 0.25) (layer "B.Cu") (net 21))
 (segment (start 147.32 85.022081) (end 147.32 71.12) (width 0.25) (layer "B.Cu") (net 22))
 (segment (start 156.277919 93.98) (end 147.32 85.022081) (width 0.25) (layer "B.Cu") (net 22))
 (segment (start 157.48 93.98) (end 156.277919 93.98) (width 0.25) (layer "B.Cu") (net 22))
 (segment (start 147.32 71.12) (end 145.796 69.596) (width 0.25) (layer "B.Cu") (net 22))
 (segment (start 145.796 69.596) (end 145.796 68.58) (width 0.25) (layer "B.Cu") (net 22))
 (segment (start 136.6 99.06) (end 134.62 99.06) (width 0.25) (layer "F.Cu") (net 23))
 (segment (start 134.62 93.98) (end 134.62 99.06) (width 0.25) (layer "F.Cu") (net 23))
 (segment (start 134.62 99.06) (end 134.62 114.3) (width 0.25) (layer "F.Cu") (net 23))
 (segment (start 134.62 114.3) (end 144.78 114.3) (width 0.25) (layer "F.Cu") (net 23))
 (segment (start 144.78 109.22) (end 144.78 114.3) (width 0.25) (layer "F.Cu") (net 23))
 (segment (start 136.6 104.14) (end 134.62 104.14) (width 0.25) (layer "F.Cu") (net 23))
 (segment (start 154.94 109.22) (end 144.78 109.22) (width 0.25) (layer "F.Cu") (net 23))
 (segment (start 144.78 114.3) (end 144.78 116.84) (width 0.25) (layer "F.Cu") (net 23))
 (segment (start 154.94 104.14) (end 157.48 104.14) (width 0.25) (layer "F.Cu") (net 24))
 (segment (start 161.835 104.14) (end 165.1 104.14) (width 0.25) (layer "F.Cu") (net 24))
 (segment (start 165.1 104.14) (end 165.1 116.84) (width 0.25) (layer "F.Cu") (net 24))
 (via (at 161.835 104.14) (size 0.8) (drill 0.4) (layers "F.Cu" "B.Cu") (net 24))
 (via (at 157.48 104.14) (size 0.8) (drill 0.4) (layers "F.Cu" "B.Cu") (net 24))
 (segment (start 157.48 104.14) (end 161.835 104.14) (width 0.25) (layer "B.Cu") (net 24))
 (segment (start 139.7 99.06) (end 139.7 93.98) (width 0.25) (layer "F.Cu") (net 29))
 (segment (start 132.08 86.36) (end 132.08 75.184) (width 0.25) (layer "F.Cu") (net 29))
 (segment (start 134.62 88.9) (end 132.08 86.36) (width 0.25) (layer "F.Cu") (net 29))
 (segment (start 132.08 75.184) (end 125.476 68.58) (width 0.25) (layer "F.Cu") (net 29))
 (segment (start 139.7 93.98) (end 134.62 88.9) (width 0.25) (layer "F.Cu") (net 29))
 (segment (start 134.62 75.184) (end 128.016 68.58) (width 0.25) (layer "F.Cu") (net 25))
 (segment (start 140.675 92.415) (end 134.62 86.36) (width 0.25) (layer "F.Cu") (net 25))
 (segment (start 139.7 104.14) (end 140.675 103.165) (width 0.25) (layer "F.Cu") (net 25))
 (segment (start 134.62 86.36) (end 134.62 75.184) (width 0.25) (layer "F.Cu") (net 25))
 (segment (start 140.675 103.165) (end 140.675 92.415) (width 0.25) (layer "F.Cu") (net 25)))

